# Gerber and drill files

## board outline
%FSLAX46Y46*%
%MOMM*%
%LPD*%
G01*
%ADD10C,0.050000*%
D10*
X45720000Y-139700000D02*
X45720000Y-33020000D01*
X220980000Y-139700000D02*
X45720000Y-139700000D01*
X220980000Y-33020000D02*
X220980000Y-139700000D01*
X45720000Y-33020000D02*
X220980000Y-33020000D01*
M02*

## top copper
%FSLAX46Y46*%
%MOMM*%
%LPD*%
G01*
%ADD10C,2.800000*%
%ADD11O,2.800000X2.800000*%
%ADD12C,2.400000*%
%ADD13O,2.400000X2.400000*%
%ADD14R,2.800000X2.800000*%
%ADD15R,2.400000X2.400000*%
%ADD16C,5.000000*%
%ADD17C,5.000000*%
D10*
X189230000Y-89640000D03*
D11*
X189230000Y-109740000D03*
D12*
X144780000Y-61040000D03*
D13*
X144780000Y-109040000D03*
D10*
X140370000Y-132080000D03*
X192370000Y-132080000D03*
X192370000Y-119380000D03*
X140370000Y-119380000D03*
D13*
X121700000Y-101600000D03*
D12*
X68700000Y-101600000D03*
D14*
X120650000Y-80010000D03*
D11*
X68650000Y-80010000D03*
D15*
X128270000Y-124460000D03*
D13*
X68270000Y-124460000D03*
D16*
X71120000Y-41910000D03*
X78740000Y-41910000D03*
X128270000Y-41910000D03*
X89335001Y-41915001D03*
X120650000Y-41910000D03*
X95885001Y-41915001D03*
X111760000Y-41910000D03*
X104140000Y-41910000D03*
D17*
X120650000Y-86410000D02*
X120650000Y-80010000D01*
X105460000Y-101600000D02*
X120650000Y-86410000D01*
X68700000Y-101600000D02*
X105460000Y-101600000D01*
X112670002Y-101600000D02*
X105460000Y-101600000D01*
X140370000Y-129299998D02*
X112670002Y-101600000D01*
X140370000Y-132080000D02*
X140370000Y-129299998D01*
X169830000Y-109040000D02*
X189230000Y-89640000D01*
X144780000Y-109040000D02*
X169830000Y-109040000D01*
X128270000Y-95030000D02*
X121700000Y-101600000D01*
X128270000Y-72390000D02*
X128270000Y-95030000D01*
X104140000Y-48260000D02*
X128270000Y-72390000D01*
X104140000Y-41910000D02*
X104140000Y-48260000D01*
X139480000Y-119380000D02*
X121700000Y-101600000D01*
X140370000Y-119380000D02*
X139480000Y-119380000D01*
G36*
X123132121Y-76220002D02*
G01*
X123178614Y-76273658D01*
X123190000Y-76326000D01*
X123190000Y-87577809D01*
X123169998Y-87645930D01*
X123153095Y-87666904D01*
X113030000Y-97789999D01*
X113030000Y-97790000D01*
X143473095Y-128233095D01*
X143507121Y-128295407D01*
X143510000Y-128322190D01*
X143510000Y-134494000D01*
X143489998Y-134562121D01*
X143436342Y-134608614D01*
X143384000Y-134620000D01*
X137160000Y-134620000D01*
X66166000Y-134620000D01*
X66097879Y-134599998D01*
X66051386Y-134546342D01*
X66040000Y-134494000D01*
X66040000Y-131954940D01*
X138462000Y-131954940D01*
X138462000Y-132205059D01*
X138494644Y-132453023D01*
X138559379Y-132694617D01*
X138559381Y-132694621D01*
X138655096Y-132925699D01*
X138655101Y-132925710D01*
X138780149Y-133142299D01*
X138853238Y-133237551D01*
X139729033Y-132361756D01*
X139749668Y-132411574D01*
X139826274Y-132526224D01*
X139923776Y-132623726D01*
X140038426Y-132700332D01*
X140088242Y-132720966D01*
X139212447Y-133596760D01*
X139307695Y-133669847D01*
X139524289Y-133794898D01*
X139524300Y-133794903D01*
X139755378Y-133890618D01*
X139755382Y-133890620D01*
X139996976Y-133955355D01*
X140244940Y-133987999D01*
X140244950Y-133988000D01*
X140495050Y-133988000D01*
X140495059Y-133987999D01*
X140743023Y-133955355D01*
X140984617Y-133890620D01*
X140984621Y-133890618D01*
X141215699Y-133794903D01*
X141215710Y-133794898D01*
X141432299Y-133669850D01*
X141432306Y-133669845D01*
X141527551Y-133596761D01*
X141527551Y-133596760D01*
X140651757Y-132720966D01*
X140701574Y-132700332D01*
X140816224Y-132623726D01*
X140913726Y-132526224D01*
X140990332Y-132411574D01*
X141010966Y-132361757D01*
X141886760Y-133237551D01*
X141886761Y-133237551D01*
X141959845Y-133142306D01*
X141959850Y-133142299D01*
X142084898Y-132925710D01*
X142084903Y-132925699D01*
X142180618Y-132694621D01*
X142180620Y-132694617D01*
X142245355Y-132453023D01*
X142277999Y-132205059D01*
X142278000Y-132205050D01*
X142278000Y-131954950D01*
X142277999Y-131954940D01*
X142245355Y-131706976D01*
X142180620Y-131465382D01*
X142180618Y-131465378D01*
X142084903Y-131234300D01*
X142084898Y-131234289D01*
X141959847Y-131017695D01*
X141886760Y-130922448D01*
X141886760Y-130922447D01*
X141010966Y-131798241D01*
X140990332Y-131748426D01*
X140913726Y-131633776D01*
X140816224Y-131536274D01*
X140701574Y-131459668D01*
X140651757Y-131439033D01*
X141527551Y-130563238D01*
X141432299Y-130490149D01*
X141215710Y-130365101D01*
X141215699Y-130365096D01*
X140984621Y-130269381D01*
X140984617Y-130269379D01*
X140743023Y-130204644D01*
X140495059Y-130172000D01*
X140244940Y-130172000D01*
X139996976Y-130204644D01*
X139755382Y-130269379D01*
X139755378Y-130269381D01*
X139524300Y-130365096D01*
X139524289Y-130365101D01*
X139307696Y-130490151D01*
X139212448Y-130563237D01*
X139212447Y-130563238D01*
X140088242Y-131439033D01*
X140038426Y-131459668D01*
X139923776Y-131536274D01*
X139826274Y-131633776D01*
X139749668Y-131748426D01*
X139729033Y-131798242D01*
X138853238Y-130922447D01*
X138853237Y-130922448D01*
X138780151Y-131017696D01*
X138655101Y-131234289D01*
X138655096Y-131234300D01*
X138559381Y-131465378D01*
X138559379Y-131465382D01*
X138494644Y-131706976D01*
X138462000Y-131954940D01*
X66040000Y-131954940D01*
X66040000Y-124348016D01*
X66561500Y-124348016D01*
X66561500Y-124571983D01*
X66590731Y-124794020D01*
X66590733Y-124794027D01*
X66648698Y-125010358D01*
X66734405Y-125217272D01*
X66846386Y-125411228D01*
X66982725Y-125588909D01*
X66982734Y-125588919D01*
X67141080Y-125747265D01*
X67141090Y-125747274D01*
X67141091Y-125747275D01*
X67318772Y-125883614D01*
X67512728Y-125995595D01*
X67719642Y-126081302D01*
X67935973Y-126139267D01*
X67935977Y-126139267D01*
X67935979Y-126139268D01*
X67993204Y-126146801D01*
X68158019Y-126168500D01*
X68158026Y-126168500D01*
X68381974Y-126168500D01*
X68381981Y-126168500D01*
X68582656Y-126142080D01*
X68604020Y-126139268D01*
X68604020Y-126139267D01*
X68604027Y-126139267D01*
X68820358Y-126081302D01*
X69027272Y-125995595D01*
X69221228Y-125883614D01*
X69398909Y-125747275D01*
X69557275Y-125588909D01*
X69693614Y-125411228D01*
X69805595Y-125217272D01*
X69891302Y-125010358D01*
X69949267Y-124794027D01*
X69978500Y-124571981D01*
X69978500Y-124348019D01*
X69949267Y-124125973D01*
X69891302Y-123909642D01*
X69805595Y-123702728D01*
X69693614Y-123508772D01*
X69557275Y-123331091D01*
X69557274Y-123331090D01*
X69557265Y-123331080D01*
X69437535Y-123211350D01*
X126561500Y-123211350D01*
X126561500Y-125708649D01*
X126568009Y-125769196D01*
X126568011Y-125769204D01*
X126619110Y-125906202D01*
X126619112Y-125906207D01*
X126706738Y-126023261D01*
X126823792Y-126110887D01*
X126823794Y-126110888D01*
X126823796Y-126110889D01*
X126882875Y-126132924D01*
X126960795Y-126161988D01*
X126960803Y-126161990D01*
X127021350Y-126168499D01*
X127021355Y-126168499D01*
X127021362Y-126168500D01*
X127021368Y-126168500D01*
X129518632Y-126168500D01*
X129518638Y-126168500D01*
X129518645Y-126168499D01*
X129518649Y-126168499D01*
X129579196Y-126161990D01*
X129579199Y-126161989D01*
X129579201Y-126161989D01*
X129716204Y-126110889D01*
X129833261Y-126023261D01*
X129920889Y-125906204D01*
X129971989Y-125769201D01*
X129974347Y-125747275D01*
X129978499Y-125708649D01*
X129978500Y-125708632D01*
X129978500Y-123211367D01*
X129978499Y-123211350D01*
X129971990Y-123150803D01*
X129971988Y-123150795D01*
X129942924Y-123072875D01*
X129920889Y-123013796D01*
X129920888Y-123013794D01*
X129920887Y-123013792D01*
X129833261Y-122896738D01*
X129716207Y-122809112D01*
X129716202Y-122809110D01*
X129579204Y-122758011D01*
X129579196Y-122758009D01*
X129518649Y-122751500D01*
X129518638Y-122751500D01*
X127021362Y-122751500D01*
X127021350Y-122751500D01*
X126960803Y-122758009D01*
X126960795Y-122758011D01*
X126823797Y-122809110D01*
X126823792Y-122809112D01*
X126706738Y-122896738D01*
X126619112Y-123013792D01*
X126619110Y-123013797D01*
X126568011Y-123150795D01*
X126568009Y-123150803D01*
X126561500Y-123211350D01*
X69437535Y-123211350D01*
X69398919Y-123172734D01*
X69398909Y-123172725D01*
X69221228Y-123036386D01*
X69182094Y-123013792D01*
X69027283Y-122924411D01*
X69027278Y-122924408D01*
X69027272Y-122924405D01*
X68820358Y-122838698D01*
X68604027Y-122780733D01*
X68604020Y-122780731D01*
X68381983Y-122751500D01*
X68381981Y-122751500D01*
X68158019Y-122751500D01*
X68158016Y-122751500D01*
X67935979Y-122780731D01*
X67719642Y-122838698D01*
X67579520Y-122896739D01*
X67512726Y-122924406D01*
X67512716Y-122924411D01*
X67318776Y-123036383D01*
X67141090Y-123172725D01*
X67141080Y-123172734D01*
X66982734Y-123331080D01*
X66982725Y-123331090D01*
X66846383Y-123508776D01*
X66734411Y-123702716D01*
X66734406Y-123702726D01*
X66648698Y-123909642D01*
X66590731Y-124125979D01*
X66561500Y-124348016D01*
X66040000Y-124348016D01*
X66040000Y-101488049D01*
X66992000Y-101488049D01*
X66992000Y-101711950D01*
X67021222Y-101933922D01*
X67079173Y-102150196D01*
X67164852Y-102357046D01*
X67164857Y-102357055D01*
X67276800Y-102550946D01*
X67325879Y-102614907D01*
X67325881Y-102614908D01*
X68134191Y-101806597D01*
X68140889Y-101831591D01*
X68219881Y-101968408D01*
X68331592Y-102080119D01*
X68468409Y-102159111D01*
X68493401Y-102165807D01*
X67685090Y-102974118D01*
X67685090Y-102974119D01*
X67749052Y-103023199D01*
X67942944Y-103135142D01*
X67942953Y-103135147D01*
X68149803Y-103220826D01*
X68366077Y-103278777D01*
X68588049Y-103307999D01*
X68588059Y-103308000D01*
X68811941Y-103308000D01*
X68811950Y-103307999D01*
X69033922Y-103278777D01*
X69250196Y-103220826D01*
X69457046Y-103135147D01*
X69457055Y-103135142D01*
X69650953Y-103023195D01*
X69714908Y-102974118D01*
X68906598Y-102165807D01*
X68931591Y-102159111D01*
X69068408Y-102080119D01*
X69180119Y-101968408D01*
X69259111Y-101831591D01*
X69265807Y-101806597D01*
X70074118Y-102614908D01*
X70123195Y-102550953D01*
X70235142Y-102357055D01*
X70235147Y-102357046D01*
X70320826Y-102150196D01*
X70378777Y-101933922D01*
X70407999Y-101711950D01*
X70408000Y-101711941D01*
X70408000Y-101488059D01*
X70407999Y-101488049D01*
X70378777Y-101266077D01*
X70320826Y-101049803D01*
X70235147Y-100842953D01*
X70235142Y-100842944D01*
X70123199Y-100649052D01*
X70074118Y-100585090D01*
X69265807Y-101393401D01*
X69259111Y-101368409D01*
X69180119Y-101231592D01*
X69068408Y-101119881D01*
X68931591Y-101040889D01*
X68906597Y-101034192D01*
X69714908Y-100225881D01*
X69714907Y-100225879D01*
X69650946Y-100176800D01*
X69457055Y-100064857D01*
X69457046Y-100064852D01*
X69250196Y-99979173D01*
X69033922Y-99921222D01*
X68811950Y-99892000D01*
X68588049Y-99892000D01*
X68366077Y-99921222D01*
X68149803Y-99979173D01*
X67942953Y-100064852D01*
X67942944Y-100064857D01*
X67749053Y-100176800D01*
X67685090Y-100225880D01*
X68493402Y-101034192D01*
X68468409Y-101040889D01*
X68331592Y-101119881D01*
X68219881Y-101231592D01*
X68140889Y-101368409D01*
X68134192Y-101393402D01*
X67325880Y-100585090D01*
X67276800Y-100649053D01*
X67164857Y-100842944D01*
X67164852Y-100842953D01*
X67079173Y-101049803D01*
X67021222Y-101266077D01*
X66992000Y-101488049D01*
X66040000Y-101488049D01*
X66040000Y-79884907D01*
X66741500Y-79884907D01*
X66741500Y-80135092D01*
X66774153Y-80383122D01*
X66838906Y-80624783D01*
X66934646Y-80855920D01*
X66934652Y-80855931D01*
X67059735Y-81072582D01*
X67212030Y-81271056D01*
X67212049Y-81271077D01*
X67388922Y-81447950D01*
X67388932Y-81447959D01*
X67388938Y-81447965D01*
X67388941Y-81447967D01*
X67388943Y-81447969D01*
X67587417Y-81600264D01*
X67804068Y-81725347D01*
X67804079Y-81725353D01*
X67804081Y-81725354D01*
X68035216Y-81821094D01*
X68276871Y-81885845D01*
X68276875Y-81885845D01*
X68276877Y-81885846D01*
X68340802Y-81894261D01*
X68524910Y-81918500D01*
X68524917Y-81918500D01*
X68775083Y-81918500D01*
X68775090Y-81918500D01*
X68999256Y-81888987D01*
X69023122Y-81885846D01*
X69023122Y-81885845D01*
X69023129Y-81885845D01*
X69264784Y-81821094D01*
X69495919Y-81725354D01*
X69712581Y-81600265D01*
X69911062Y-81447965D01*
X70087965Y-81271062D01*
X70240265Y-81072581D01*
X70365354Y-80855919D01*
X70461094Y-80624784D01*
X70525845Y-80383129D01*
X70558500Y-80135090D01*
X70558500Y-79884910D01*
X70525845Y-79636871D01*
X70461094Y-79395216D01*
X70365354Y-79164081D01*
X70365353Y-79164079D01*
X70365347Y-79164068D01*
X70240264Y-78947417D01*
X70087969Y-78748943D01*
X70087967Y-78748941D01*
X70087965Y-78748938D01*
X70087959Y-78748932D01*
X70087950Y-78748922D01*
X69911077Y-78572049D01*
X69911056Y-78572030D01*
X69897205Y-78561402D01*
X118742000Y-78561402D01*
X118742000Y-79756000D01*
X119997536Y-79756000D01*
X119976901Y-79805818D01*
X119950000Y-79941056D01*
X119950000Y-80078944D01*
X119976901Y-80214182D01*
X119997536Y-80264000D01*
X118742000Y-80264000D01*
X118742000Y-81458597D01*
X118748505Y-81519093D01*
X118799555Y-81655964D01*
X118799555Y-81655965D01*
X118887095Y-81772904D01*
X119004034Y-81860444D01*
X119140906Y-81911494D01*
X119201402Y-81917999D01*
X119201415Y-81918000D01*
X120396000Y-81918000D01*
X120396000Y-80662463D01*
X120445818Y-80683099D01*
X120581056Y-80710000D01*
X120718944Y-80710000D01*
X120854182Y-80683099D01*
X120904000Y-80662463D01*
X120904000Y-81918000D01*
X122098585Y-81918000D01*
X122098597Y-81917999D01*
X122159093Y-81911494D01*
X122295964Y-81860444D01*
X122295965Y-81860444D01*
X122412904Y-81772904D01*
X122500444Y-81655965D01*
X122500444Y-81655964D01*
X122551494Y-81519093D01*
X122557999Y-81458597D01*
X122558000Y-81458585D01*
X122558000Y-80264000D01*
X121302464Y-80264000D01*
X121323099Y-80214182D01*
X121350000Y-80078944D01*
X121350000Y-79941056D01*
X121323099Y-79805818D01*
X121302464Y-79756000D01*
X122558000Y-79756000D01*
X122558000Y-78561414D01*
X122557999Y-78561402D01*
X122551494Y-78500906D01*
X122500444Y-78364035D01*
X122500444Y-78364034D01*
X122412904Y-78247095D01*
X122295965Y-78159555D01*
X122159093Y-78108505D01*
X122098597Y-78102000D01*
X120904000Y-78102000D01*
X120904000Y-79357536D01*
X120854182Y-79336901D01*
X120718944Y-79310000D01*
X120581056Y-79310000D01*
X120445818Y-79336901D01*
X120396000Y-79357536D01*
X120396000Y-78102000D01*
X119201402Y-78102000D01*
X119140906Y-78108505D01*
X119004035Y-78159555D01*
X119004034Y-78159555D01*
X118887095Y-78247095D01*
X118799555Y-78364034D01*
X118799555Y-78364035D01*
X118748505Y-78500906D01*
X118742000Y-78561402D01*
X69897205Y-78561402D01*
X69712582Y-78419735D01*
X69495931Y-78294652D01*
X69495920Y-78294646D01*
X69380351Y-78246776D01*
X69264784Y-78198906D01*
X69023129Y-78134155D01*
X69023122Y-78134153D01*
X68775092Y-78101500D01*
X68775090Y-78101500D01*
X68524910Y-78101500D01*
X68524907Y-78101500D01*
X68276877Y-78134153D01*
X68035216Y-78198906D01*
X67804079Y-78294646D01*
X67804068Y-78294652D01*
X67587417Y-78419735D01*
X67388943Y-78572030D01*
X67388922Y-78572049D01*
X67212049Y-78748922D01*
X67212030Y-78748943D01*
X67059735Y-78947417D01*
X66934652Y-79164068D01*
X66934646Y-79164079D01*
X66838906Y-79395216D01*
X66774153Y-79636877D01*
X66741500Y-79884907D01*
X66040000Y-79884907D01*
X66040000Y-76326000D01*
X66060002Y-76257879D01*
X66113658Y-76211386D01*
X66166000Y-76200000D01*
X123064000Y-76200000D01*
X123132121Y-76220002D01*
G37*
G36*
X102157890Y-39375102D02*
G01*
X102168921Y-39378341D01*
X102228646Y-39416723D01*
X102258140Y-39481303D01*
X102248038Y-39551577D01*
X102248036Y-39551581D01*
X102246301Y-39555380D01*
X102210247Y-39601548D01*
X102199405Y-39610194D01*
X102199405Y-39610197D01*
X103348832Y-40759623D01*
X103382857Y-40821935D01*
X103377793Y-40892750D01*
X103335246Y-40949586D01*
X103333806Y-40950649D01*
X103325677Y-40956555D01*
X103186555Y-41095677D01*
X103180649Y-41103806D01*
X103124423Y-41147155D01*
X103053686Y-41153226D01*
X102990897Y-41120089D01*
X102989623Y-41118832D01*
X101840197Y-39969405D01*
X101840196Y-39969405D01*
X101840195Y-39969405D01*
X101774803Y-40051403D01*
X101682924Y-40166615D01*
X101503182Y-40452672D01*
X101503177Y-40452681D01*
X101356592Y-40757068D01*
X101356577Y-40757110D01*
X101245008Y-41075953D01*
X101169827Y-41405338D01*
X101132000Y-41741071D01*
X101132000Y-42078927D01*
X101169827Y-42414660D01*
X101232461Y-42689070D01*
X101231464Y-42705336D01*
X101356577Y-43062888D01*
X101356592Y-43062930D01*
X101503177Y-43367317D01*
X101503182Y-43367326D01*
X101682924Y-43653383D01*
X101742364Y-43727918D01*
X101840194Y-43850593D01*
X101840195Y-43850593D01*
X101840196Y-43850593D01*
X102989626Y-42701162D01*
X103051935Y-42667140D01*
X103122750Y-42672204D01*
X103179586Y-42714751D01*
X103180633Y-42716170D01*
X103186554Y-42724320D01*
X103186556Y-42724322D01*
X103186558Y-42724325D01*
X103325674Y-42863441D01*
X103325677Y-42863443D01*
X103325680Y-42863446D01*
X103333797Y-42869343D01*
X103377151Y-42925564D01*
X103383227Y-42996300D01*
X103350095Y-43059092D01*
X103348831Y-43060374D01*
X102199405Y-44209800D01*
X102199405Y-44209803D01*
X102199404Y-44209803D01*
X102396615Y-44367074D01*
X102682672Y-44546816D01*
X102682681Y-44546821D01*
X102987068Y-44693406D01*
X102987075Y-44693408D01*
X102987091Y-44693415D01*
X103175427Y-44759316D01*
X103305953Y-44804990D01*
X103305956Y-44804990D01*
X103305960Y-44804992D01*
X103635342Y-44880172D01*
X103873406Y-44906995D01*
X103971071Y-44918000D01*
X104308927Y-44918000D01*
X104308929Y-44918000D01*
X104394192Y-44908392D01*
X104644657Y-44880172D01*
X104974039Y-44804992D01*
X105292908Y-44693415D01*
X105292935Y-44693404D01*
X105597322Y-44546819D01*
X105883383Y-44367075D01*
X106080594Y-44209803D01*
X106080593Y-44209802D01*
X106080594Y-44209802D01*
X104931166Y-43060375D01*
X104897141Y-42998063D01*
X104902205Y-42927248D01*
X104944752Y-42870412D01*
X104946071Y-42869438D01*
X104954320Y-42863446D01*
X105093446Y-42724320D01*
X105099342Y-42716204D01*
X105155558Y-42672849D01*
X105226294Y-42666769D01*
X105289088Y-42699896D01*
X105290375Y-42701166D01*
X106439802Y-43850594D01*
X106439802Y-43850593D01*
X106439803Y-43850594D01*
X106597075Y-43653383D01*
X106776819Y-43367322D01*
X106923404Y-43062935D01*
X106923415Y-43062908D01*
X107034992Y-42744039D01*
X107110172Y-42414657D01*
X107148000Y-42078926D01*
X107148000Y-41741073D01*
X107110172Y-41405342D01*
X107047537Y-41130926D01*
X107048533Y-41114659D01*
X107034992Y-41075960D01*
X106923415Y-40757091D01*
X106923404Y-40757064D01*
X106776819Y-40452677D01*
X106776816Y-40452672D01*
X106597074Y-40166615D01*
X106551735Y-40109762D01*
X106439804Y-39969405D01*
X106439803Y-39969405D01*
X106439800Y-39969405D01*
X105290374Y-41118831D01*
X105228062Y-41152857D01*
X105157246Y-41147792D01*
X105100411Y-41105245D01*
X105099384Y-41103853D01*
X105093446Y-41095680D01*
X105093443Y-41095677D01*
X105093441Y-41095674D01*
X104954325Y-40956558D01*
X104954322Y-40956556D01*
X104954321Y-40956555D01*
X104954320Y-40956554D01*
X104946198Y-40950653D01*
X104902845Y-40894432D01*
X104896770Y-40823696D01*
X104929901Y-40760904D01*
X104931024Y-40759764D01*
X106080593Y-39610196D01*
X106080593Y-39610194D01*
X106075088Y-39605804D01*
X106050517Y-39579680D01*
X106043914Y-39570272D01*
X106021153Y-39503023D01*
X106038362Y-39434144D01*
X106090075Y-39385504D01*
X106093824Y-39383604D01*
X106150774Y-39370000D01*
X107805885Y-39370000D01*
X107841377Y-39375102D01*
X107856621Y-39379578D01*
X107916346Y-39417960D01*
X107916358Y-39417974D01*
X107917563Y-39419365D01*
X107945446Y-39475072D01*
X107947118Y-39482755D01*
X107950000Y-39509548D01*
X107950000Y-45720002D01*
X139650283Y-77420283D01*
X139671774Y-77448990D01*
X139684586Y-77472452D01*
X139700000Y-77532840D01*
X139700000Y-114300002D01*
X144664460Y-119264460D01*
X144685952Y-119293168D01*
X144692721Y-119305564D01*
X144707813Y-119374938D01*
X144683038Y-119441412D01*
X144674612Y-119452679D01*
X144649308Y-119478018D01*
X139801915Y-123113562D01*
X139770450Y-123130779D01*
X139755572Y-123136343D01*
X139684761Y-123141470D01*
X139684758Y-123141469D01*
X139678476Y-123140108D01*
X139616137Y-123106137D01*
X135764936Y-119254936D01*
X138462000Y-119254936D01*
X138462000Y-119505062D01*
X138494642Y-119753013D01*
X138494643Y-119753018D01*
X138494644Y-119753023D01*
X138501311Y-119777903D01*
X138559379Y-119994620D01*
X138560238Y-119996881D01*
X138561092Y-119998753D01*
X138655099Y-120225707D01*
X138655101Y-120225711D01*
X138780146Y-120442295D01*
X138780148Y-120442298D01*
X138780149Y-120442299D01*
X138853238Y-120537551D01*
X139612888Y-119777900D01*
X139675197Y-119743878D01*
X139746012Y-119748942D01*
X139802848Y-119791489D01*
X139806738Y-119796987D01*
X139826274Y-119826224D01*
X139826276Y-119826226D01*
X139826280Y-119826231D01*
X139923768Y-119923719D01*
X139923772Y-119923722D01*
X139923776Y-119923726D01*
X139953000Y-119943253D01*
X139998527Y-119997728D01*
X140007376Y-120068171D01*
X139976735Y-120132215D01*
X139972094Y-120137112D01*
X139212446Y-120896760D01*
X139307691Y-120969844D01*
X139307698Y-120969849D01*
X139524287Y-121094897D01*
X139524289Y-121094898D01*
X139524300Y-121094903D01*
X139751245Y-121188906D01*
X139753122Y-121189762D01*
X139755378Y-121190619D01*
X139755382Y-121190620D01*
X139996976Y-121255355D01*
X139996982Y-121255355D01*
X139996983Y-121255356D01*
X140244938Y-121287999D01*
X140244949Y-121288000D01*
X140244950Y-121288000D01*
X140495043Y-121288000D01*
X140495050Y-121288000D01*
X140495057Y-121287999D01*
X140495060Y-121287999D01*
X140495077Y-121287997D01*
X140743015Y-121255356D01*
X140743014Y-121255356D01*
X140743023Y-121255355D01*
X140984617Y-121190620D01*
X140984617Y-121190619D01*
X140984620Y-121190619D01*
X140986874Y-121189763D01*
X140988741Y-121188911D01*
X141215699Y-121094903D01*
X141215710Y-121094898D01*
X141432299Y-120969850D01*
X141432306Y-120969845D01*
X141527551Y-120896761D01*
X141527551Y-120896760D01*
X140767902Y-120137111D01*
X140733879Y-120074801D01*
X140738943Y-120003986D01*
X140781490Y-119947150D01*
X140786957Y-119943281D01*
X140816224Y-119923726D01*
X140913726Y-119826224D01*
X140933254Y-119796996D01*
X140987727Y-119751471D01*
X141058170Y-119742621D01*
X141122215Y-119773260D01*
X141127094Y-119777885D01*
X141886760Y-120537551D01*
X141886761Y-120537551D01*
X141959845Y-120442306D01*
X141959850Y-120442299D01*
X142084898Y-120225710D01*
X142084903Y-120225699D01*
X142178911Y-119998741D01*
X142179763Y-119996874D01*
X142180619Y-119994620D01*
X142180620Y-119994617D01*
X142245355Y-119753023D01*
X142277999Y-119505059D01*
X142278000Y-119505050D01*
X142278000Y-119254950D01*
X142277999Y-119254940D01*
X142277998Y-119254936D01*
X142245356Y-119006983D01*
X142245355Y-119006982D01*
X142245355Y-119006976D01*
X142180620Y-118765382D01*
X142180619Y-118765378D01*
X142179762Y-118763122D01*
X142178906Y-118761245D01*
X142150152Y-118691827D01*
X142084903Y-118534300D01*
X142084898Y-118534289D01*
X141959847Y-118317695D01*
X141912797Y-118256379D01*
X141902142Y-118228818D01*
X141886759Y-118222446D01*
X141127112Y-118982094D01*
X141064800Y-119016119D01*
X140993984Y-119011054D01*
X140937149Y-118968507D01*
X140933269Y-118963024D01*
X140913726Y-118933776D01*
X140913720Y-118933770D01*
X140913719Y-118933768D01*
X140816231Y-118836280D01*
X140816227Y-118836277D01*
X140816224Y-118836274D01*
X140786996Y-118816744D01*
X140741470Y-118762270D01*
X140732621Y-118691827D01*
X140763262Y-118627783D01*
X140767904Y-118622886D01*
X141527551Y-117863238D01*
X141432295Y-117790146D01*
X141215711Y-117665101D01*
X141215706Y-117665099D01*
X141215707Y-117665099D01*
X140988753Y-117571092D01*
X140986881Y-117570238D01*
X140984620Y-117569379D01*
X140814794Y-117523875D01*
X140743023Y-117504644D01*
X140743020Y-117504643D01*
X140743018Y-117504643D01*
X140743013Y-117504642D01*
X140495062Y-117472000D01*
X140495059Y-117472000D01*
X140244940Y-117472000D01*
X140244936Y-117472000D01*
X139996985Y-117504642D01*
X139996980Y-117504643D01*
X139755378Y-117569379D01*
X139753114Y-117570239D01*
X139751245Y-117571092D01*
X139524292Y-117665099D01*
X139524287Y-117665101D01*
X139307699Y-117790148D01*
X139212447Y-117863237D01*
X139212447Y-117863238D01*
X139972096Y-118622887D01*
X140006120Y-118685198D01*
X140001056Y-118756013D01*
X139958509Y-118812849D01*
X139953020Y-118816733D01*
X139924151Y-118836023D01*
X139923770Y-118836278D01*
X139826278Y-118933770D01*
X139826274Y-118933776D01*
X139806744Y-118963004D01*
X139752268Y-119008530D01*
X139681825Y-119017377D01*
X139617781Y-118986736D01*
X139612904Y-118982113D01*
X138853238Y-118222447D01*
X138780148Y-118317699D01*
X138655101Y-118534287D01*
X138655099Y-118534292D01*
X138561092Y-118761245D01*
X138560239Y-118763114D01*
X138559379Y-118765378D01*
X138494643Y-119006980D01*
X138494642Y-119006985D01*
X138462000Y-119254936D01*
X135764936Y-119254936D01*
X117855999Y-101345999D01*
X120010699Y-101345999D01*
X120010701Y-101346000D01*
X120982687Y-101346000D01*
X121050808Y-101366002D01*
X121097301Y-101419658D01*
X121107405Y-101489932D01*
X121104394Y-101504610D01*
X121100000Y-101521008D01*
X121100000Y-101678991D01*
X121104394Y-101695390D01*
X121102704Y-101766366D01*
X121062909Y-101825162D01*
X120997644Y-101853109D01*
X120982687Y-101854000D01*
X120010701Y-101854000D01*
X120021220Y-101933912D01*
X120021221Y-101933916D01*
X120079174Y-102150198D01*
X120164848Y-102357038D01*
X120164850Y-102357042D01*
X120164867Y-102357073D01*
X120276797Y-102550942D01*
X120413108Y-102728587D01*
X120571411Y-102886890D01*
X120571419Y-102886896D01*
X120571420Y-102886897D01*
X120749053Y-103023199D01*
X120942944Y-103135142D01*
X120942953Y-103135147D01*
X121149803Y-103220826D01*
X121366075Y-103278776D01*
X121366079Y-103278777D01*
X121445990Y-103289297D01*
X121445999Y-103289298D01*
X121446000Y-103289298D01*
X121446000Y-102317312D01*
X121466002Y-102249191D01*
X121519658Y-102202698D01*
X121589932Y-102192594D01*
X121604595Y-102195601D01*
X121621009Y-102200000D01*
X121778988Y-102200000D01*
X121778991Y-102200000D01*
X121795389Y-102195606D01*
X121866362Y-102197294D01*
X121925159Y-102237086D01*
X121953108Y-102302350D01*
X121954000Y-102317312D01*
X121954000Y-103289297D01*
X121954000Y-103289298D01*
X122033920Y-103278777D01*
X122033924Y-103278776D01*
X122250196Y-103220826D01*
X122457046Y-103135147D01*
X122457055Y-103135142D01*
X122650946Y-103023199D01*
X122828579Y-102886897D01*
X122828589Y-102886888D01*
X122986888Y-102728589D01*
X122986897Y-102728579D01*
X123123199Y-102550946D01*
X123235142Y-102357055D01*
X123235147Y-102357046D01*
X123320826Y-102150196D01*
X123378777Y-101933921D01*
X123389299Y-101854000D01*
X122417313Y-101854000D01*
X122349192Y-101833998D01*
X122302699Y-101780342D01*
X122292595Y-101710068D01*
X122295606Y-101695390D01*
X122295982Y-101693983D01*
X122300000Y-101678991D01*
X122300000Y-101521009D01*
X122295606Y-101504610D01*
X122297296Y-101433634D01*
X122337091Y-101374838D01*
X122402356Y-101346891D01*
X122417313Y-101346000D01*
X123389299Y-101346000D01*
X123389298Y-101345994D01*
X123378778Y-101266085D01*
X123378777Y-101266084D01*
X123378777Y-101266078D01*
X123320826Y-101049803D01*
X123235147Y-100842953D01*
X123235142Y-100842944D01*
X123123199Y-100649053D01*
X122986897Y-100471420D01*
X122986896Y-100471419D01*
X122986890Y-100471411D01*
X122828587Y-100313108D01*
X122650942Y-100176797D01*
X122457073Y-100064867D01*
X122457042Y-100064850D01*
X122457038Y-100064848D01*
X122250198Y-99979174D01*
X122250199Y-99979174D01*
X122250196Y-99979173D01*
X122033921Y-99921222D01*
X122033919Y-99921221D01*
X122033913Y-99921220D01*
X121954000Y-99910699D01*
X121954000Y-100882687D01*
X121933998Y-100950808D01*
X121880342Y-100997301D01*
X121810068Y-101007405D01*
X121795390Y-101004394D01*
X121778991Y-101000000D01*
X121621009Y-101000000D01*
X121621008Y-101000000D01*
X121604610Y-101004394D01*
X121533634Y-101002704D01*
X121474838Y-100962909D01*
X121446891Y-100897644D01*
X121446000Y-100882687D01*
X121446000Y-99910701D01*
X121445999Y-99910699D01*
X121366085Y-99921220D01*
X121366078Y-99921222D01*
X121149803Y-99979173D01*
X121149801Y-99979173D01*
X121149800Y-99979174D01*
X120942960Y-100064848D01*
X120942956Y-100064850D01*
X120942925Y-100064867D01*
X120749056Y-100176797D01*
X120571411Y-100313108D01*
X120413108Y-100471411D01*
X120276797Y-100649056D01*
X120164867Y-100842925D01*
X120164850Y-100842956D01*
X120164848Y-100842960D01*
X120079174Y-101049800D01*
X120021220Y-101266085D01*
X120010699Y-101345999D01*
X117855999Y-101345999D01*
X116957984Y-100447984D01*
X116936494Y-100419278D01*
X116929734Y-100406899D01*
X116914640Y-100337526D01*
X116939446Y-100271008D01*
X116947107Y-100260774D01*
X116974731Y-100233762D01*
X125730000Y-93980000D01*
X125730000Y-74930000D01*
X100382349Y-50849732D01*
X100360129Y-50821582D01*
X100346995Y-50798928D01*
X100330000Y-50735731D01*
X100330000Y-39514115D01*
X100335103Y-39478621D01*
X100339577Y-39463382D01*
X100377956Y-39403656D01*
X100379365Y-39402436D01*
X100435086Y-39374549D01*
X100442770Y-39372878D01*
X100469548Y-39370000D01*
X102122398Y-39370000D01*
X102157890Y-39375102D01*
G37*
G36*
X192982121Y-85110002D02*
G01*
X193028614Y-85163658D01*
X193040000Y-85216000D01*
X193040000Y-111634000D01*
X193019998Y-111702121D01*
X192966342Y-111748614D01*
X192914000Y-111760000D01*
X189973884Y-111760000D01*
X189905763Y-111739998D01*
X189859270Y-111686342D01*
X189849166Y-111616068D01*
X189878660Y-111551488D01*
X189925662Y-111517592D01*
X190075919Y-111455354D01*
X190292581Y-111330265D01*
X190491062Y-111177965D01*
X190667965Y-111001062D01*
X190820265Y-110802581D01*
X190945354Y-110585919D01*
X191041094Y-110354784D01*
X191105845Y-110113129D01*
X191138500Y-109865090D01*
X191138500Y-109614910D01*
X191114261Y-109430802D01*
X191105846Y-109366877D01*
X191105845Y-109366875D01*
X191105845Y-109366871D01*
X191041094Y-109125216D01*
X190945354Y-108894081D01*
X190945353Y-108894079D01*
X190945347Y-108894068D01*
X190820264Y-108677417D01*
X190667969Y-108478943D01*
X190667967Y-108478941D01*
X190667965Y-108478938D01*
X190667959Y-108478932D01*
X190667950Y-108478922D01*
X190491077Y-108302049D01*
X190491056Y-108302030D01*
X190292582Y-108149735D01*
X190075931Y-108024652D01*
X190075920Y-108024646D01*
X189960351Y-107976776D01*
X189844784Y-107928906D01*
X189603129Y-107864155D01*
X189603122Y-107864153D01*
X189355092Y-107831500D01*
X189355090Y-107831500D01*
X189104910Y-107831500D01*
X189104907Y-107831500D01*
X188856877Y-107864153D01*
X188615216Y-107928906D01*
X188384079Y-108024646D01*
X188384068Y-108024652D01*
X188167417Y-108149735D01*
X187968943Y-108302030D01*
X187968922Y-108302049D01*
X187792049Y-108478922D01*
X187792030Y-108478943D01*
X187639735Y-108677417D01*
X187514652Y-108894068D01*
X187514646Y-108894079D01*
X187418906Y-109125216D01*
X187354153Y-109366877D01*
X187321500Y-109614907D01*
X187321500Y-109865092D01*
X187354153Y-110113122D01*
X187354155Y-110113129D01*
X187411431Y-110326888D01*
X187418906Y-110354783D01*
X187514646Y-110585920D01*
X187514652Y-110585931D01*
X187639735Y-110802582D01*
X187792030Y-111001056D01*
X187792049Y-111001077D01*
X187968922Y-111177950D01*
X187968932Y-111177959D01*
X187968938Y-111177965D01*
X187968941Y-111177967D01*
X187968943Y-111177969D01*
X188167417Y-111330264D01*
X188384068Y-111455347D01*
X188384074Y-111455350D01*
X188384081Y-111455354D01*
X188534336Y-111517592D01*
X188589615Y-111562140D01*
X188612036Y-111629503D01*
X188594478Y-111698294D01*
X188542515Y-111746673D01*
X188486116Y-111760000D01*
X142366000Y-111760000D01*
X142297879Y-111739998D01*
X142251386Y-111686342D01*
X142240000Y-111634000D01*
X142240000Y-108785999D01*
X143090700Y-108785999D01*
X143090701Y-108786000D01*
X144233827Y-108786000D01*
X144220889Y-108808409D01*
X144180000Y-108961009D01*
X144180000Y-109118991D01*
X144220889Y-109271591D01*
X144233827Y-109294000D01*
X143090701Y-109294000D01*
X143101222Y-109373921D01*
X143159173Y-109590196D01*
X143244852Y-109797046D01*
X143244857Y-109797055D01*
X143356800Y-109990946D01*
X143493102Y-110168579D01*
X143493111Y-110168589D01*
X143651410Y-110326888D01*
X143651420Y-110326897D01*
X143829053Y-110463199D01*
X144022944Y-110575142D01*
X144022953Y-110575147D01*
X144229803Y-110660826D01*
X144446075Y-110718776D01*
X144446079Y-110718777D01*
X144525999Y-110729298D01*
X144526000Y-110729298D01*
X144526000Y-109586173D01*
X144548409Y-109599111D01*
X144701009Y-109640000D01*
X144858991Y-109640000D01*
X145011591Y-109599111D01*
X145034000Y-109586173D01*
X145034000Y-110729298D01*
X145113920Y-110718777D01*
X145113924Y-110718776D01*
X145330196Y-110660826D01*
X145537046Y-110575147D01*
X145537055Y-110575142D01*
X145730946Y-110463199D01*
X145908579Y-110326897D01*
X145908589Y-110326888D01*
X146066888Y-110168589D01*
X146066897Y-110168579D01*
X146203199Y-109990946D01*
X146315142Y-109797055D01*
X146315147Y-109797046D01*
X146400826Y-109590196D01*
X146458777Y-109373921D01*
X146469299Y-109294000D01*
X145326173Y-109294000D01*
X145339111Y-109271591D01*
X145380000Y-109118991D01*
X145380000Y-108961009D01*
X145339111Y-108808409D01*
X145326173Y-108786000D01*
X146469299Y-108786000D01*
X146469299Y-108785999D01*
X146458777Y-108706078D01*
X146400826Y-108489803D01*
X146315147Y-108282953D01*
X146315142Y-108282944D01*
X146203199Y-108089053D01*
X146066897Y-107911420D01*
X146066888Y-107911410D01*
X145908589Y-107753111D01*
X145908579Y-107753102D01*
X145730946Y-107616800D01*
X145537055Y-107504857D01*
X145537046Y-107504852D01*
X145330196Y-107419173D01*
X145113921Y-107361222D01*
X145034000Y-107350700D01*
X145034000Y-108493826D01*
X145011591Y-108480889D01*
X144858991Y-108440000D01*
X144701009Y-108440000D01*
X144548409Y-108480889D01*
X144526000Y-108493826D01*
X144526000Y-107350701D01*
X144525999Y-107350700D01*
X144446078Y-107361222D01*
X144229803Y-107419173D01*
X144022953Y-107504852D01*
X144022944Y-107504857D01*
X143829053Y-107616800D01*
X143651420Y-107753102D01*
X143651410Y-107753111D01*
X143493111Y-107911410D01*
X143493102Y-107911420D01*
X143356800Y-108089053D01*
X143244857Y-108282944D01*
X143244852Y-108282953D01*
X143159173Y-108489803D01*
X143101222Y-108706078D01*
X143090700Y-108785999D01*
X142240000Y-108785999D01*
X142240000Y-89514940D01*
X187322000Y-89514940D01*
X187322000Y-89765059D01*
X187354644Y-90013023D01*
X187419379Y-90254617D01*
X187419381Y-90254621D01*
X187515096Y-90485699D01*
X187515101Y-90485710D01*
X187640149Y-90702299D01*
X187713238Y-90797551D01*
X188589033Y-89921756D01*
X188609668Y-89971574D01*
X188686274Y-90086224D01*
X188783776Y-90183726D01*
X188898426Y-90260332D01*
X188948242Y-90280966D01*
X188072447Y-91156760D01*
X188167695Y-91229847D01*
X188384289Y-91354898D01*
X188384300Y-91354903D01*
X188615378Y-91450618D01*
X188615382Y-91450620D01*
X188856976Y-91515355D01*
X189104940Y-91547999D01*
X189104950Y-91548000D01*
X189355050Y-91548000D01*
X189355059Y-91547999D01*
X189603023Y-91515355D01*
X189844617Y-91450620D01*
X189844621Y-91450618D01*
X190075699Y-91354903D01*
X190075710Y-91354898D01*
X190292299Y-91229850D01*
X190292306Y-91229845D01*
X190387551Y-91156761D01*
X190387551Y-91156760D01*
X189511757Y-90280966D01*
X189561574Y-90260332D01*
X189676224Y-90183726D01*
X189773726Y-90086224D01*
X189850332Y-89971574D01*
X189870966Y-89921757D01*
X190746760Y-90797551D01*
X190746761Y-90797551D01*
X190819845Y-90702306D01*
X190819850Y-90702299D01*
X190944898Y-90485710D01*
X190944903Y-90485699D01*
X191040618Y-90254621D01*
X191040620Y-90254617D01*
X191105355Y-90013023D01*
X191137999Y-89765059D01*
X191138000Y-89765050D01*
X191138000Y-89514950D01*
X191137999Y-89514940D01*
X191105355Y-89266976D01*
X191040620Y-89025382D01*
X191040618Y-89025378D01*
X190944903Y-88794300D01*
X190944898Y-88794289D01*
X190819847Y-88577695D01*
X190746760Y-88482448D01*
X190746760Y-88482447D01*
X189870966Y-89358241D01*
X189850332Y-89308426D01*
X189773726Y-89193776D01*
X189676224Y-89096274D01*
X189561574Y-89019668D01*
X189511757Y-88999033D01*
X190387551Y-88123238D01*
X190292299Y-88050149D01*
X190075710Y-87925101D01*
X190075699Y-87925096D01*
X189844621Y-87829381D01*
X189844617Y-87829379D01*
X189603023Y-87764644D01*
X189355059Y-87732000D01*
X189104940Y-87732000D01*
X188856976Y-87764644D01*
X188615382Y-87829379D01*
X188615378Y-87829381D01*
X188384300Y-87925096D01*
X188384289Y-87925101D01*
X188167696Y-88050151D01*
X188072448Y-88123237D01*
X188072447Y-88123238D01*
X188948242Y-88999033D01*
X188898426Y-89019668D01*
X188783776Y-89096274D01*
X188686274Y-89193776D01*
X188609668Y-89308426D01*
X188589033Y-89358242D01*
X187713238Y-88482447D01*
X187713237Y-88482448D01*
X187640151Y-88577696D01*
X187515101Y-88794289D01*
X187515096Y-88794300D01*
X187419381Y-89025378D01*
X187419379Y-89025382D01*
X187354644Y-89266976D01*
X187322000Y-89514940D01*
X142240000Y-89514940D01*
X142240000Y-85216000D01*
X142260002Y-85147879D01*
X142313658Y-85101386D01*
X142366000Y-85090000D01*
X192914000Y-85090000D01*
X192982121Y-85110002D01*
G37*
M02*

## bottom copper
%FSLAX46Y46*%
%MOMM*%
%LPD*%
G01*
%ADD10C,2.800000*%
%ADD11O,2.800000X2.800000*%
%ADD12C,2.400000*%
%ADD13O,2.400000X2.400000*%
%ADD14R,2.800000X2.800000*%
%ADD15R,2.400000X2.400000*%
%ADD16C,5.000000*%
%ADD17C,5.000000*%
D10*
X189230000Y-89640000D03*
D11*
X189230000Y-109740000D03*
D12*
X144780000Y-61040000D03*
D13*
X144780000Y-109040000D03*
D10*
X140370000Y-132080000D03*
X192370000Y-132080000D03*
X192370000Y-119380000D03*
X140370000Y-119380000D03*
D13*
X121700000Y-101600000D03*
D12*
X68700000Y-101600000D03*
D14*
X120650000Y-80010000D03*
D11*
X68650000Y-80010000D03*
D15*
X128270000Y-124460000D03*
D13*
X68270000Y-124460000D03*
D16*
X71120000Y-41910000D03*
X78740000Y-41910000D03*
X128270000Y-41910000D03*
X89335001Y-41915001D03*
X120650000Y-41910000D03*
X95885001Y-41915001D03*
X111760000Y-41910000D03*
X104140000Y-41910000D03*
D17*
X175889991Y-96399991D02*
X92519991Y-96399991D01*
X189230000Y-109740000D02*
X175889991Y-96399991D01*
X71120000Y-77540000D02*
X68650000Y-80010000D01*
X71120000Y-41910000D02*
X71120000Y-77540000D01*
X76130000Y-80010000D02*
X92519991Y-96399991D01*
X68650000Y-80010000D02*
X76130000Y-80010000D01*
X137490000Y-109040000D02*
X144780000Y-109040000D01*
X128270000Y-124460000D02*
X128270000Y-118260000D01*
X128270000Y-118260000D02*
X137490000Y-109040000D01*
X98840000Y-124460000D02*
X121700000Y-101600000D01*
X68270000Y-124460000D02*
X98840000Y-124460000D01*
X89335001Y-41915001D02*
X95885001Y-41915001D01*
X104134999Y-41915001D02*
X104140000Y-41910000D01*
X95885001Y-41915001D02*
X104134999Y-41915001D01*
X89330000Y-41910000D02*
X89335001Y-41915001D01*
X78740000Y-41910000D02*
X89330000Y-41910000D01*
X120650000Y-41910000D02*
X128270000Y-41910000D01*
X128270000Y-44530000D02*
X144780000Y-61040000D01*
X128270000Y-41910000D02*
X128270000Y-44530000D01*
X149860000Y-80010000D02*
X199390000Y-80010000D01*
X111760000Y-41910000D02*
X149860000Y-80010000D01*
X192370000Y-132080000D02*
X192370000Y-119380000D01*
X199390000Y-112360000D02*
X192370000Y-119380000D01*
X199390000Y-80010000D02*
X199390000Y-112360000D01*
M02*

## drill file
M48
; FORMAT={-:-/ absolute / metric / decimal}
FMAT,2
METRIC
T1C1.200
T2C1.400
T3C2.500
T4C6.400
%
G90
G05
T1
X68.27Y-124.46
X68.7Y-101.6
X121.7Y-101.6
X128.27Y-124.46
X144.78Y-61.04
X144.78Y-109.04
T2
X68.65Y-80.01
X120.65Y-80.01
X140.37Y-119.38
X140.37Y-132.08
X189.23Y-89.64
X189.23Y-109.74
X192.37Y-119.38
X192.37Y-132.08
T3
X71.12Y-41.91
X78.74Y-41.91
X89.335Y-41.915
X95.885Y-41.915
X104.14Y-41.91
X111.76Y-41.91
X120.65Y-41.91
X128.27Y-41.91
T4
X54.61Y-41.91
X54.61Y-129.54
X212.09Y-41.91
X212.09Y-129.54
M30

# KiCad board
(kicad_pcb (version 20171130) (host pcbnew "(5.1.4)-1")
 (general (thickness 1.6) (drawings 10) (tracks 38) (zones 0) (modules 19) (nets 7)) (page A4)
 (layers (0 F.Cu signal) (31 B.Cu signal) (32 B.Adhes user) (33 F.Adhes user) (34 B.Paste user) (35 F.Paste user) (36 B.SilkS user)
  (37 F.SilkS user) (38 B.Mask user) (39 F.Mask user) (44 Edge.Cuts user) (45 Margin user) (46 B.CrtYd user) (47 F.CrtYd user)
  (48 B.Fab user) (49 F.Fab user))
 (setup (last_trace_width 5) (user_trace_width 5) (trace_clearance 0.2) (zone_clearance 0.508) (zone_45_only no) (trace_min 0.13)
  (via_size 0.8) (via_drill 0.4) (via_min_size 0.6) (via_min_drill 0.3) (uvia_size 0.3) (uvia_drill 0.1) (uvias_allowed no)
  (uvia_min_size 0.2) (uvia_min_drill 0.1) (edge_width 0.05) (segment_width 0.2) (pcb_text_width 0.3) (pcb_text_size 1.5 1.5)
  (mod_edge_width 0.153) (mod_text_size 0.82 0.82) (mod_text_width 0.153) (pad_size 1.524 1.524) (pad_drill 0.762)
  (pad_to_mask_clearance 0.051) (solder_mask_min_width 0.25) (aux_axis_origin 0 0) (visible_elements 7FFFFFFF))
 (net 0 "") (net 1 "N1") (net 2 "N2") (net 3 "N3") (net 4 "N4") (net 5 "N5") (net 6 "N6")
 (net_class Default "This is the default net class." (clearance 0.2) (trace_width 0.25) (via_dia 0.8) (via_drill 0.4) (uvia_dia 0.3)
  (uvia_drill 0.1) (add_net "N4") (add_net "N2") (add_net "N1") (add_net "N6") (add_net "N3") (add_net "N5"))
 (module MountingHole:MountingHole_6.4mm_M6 (layer F.Cu) (at 212.09 41.91)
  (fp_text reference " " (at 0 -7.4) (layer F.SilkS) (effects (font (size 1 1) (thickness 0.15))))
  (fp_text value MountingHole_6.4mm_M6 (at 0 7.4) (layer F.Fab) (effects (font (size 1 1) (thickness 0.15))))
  (pad 1 np_thru_hole circle (at 0 0) (size 6.4 6.4) (drill 6.4) (layers *.Cu *.Mask)))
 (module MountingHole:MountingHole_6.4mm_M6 (layer F.Cu) (at 54.61 129.54)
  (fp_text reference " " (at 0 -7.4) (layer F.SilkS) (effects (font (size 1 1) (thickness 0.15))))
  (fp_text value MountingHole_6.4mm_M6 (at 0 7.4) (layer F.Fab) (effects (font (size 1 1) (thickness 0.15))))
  (pad 1 np_thru_hole circle (at 0 0) (size 6.4 6.4) (drill 6.4) (layers *.Cu *.Mask)))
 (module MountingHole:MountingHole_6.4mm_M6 (layer F.Cu) (at 54.61 41.91)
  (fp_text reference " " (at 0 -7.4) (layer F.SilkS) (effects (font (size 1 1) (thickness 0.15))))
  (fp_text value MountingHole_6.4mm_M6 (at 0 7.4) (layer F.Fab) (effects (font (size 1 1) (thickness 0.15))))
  (pad 1 np_thru_hole circle (at 0 0) (size 6.4 6.4) (drill 6.4) (layers *.Cu *.Mask)))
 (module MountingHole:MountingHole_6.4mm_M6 (layer F.Cu) (at 212.09 129.54)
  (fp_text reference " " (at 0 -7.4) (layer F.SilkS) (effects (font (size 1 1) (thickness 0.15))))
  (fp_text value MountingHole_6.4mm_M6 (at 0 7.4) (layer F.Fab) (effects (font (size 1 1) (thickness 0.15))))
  (pad 1 np_thru_hole circle (at 0 0) (size 6.4 6.4) (drill 6.4) (layers *.Cu *.Mask)))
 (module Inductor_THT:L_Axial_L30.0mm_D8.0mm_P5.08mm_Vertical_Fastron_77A (layer F.Cu) (at 189.23 78.74 270)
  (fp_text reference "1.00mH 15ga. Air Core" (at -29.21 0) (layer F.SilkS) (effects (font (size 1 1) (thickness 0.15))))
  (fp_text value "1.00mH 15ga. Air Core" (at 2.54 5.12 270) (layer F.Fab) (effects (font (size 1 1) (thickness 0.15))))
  (pad 1 thru_hole circle (at 10.9 0 270) (size 2.8 2.8) (drill 1.4) (layers *.Cu *.Mask) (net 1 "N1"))
  (pad 2 thru_hole oval (at 31 0 270) (size 2.8 2.8) (drill 1.4) (layers *.Cu *.Mask) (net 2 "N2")))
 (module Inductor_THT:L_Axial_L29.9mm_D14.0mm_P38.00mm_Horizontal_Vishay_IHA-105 (layer F.Cu) (at 144.78 66.04 270)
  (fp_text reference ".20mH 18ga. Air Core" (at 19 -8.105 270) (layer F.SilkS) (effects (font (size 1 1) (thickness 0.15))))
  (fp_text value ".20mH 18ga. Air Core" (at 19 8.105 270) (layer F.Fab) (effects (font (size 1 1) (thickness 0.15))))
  (pad 1 thru_hole circle (at -5 0 270) (size 2.4 2.4) (drill 1.2) (layers *.Cu *.Mask) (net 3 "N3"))
  (pad 2 thru_hole oval (at 43 0 270) (size 2.4 2.4) (drill 1.2) (layers *.Cu *.Mask) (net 1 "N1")))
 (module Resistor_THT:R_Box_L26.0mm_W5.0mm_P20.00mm (layer F.Cu) (at 166.37 132.08 180)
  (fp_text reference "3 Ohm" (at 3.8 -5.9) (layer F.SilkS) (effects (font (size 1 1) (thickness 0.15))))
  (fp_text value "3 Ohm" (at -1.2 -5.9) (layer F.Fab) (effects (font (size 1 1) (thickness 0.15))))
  (pad 2 thru_hole circle (at 26 0 180) (size 2.8 2.8) (drill 1.4) (layers *.Cu *.Mask) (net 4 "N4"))
  (pad 1 thru_hole circle (at -26 0 180) (size 2.8 2.8) (drill 1.4) (layers *.Cu *.Mask) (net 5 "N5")))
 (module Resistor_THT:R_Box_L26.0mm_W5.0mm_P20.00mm (layer F.Cu) (at 166.37 119.38)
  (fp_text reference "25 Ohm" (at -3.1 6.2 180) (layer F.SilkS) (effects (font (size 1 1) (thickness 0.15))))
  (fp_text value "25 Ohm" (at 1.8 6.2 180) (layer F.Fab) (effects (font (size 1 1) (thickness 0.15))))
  (pad 2 thru_hole circle (at 26 0) (size 2.8 2.8) (drill 1.4) (layers *.Cu *.Mask) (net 5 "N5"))
  (pad 1 thru_hole circle (at -26 0) (size 2.8 2.8) (drill 1.4) (layers *.Cu *.Mask) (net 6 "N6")))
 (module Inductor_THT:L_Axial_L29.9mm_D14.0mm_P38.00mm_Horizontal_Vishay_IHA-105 (layer F.Cu) (at 76.2 101.6)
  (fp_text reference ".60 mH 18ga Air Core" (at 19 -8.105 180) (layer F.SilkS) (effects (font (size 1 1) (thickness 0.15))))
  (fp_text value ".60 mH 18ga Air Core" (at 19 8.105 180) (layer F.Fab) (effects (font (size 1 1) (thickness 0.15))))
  (pad 2 thru_hole oval (at 45.5 0) (size 2.4 2.4) (drill 1.2) (layers *.Cu *.Mask) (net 6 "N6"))
  (pad 1 thru_hole circle (at -7.5 0) (size 2.4 2.4) (drill 1.2) (layers *.Cu *.Mask) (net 4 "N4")))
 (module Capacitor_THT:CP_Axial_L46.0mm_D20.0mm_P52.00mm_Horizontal (layer F.Cu) (at 120.65 80.01 180)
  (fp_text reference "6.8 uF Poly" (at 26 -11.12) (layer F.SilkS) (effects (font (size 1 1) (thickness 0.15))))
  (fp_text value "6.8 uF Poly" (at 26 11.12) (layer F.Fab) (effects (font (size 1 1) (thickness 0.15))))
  (pad 1 thru_hole rect (at 0 0 180) (size 2.8 2.8) (drill 1.4) (layers *.Cu *.Mask) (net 4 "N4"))
  (pad 2 thru_hole oval (at 52 0 180) (size 2.8 2.8) (drill 1.4) (layers *.Cu *.Mask) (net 2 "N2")))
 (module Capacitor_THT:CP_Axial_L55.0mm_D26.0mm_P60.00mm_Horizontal (layer F.Cu) (at 128.27 124.46 180)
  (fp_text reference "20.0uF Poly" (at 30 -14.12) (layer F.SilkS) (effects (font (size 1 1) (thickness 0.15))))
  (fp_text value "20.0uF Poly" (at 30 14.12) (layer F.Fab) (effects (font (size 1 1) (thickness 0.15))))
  (pad 1 thru_hole rect (at 0 0 180) (size 2.4 2.4) (drill 1.2) (layers *.Cu *.Mask) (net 1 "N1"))
  (pad 2 thru_hole oval (at 60 0 180) (size 2.4 2.4) (drill 1.2) (layers *.Cu *.Mask) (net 6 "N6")))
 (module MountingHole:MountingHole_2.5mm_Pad (layer F.Cu) (at 71.12 41.91)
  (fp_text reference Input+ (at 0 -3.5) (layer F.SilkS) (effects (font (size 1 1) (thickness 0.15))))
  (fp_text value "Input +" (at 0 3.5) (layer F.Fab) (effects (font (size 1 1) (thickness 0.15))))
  (pad 1 thru_hole circle (at 0 0) (size 5 5) (drill 2.5) (layers *.Cu *.Mask) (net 2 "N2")))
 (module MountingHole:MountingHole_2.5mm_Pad (layer F.Cu) (at 78.74 41.91)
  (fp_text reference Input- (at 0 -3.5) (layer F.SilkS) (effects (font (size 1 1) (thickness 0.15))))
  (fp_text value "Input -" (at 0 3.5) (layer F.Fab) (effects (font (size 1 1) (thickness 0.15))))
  (pad 1 thru_hole circle (at 0 0) (size 5 5) (drill 2.5) (layers *.Cu *.Mask) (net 6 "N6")))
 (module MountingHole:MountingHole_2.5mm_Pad (layer F.Cu) (at 128.27 41.91)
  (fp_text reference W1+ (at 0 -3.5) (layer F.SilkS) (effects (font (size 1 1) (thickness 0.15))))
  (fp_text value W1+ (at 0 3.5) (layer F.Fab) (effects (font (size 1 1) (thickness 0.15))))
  (pad 1 thru_hole circle (at 0 0) (size 5 5) (drill 2.5) (layers *.Cu *.Mask) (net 3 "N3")))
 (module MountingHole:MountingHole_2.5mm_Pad (layer F.Cu) (at 89.335001 41.915001)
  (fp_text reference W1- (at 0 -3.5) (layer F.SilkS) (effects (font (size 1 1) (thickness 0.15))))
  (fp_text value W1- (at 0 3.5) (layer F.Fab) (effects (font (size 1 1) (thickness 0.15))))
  (pad 1 thru_hole circle (at 0 0) (size 5 5) (drill 2.5) (layers *.Cu *.Mask) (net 6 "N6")))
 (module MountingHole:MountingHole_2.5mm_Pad (layer F.Cu) (at 120.65 41.91)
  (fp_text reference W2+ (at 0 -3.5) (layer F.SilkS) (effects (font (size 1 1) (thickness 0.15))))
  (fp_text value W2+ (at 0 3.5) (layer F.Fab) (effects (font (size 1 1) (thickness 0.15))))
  (pad 1 thru_hole circle (at 0 0) (size 5 5) (drill 2.5) (layers *.Cu *.Mask) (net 3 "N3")))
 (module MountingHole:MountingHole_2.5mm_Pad (layer F.Cu) (at 95.885001 41.915001)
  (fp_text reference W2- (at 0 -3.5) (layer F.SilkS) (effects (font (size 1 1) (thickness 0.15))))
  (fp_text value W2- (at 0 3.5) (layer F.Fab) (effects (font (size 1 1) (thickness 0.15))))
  (pad 1 thru_hole circle (at 0 0) (size 5 5) (drill 2.5) (layers *.Cu *.Mask) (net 6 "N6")))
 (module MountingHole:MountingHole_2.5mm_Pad (layer F.Cu) (at 111.76 41.91)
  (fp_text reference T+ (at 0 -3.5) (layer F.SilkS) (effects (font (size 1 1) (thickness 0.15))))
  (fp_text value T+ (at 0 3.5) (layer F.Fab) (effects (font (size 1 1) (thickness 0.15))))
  (pad 1 thru_hole circle (at 0 0) (size 5 5) (drill 2.5) (layers *.Cu *.Mask) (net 5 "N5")))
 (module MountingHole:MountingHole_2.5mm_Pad (layer F.Cu) (at 104.14 41.91)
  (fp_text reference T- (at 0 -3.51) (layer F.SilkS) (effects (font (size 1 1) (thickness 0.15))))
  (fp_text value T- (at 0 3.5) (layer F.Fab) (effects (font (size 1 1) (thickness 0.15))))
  (pad 1 thru_hole circle (at 0 0) (size 5 5) (drill 2.5) (layers *.Cu *.Mask) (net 6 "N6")))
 (gr_line (start 45.72 139.7) (end 45.72 33.02) (layer Edge.Cuts) (width 0.05))
 (gr_line (start 220.98 139.7) (end 45.72 139.7) (layer Edge.Cuts) (width 0.05))
 (gr_line (start 220.98 33.02) (end 220.98 139.7) (layer Edge.Cuts) (width 0.05))
 (gr_line (start 45.72 33.02) (end 220.98 33.02) (layer Edge.Cuts) (width 0.05))
 (segment (start 120.65 86.41) (end 120.65 80.01) (width 5) (layer F.Cu) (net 4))
 (segment (start 105.46 101.6) (end 120.65 86.41) (width 5) (layer F.Cu) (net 4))
 (segment (start 68.7 101.6) (end 105.46 101.6) (width 5) (layer F.Cu) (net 4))
 (segment (start 112.670002 101.6) (end 105.46 101.6) (width 5) (layer F.Cu) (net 4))
 (segment (start 140.37 129.299998) (end 112.670002 101.6) (width 5) (layer F.Cu) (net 4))
 (segment (start 140.37 132.08) (end 140.37 129.299998) (width 5) (layer F.Cu) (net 4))
 (segment (start 175.889991 96.399991) (end 92.519991 96.399991) (width 5) (layer B.Cu) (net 2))
 (segment (start 189.23 109.74) (end 175.889991 96.399991) (width 5) (layer B.Cu) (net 2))
 (segment (start 71.12 77.54) (end 68.65 80.01) (width 5) (layer B.Cu) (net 2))
 (segment (start 71.12 41.91) (end 71.12 77.54) (width 5) (layer B.Cu) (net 2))
 (segment (start 76.13 80.01) (end 92.519991 96.399991) (width 5) (layer B.Cu) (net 2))
 (segment (start 68.65 80.01) (end 76.13 80.01) (width 5) (layer B.Cu) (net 2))
 (segment (start 137.49 109.04) (end 144.78 109.04) (width 5) (layer B.Cu) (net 1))
 (segment (start 128.27 124.46) (end 128.27 118.26) (width 5) (layer B.Cu) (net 1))
 (segment (start 128.27 118.26) (end 137.49 109.04) (width 5) (layer B.Cu) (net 1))
 (segment (start 169.83 109.04) (end 189.23 89.64) (width 5) (layer F.Cu) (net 1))
 (segment (start 144.78 109.04) (end 169.83 109.04) (width 5) (layer F.Cu) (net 1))
 (segment (start 98.84 124.46) (end 121.7 101.6) (width 5) (layer B.Cu) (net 6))
 (segment (start 68.27 124.46) (end 98.84 124.46) (width 5) (layer B.Cu) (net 6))
 (segment (start 89.335001 41.915001) (end 95.885001 41.915001) (width 5) (layer B.Cu) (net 6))
 (segment (start 104.134999 41.915001) (end 104.14 41.91) (width 5) (layer B.Cu) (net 6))
 (segment (start 95.885001 41.915001) (end 104.134999 41.915001) (width 5) (layer B.Cu) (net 6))
 (segment (start 128.27 95.03) (end 121.7 101.6) (width 5) (layer F.Cu) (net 6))
 (segment (start 128.27 72.39) (end 128.27 95.03) (width 5) (layer F.Cu) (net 6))
 (segment (start 104.14 48.26) (end 128.27 72.39) (width 5) (layer F.Cu) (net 6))
 (segment (start 104.14 41.91) (end 104.14 48.26) (width 5) (layer F.Cu) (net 6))
 (segment (start 139.48 119.38) (end 121.7 101.6) (width 5) (layer F.Cu) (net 6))
 (segment (start 140.37 119.38) (end 139.48 119.38) (width 5) (layer F.Cu) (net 6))
 (segment (start 89.33 41.91) (end 89.335001 41.915001) (width 5) (layer B.Cu) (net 6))
 (segment (start 78.74 41.91) (end 89.33 41.91) (width 5) (layer B.Cu) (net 6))
 (segment (start 120.65 41.91) (end 128.27 41.91) (width 5) (layer B.Cu) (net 3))
 (segment (start 128.27 44.53) (end 144.78 61.04) (width 5) (layer B.Cu) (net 3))
 (segment (start 128.27 41.91) (end 128.27 44.53) (width 5) (layer B.Cu) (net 3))
 (segment (start 149.86 80.01) (end 199.39 80.01) (width 5) (layer B.Cu) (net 5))
 (segment (start 111.76 41.91) (end 149.86 80.01) (width 5) (layer B.Cu) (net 5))
 (segment (start 192.37 132.08) (end 192.37 119.38) (width 5) (layer B.Cu) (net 5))
 (segment (start 199.39 112.36) (end 192.37 119.38) (width 5) (layer B.Cu) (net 5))
 (segment (start 199.39 80.01) (end 199.39 112.36) (width 5) (layer B.Cu) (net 5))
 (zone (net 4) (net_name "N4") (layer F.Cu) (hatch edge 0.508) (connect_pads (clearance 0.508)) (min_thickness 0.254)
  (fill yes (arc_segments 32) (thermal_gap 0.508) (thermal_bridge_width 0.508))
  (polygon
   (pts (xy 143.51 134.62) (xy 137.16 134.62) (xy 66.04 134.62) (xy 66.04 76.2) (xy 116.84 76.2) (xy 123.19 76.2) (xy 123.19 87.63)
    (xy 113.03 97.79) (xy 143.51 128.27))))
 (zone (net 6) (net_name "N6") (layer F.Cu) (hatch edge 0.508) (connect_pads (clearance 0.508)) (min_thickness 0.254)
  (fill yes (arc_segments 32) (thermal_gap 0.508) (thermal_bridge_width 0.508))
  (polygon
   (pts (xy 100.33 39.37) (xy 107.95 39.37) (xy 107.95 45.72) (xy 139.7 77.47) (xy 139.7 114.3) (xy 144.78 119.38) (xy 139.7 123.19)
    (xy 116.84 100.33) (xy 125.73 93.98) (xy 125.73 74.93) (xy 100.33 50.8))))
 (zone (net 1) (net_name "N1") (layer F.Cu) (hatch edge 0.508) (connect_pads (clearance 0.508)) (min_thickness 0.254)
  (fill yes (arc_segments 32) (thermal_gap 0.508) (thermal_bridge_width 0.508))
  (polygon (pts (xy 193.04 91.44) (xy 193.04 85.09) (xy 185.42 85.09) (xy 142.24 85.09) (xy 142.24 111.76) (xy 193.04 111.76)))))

